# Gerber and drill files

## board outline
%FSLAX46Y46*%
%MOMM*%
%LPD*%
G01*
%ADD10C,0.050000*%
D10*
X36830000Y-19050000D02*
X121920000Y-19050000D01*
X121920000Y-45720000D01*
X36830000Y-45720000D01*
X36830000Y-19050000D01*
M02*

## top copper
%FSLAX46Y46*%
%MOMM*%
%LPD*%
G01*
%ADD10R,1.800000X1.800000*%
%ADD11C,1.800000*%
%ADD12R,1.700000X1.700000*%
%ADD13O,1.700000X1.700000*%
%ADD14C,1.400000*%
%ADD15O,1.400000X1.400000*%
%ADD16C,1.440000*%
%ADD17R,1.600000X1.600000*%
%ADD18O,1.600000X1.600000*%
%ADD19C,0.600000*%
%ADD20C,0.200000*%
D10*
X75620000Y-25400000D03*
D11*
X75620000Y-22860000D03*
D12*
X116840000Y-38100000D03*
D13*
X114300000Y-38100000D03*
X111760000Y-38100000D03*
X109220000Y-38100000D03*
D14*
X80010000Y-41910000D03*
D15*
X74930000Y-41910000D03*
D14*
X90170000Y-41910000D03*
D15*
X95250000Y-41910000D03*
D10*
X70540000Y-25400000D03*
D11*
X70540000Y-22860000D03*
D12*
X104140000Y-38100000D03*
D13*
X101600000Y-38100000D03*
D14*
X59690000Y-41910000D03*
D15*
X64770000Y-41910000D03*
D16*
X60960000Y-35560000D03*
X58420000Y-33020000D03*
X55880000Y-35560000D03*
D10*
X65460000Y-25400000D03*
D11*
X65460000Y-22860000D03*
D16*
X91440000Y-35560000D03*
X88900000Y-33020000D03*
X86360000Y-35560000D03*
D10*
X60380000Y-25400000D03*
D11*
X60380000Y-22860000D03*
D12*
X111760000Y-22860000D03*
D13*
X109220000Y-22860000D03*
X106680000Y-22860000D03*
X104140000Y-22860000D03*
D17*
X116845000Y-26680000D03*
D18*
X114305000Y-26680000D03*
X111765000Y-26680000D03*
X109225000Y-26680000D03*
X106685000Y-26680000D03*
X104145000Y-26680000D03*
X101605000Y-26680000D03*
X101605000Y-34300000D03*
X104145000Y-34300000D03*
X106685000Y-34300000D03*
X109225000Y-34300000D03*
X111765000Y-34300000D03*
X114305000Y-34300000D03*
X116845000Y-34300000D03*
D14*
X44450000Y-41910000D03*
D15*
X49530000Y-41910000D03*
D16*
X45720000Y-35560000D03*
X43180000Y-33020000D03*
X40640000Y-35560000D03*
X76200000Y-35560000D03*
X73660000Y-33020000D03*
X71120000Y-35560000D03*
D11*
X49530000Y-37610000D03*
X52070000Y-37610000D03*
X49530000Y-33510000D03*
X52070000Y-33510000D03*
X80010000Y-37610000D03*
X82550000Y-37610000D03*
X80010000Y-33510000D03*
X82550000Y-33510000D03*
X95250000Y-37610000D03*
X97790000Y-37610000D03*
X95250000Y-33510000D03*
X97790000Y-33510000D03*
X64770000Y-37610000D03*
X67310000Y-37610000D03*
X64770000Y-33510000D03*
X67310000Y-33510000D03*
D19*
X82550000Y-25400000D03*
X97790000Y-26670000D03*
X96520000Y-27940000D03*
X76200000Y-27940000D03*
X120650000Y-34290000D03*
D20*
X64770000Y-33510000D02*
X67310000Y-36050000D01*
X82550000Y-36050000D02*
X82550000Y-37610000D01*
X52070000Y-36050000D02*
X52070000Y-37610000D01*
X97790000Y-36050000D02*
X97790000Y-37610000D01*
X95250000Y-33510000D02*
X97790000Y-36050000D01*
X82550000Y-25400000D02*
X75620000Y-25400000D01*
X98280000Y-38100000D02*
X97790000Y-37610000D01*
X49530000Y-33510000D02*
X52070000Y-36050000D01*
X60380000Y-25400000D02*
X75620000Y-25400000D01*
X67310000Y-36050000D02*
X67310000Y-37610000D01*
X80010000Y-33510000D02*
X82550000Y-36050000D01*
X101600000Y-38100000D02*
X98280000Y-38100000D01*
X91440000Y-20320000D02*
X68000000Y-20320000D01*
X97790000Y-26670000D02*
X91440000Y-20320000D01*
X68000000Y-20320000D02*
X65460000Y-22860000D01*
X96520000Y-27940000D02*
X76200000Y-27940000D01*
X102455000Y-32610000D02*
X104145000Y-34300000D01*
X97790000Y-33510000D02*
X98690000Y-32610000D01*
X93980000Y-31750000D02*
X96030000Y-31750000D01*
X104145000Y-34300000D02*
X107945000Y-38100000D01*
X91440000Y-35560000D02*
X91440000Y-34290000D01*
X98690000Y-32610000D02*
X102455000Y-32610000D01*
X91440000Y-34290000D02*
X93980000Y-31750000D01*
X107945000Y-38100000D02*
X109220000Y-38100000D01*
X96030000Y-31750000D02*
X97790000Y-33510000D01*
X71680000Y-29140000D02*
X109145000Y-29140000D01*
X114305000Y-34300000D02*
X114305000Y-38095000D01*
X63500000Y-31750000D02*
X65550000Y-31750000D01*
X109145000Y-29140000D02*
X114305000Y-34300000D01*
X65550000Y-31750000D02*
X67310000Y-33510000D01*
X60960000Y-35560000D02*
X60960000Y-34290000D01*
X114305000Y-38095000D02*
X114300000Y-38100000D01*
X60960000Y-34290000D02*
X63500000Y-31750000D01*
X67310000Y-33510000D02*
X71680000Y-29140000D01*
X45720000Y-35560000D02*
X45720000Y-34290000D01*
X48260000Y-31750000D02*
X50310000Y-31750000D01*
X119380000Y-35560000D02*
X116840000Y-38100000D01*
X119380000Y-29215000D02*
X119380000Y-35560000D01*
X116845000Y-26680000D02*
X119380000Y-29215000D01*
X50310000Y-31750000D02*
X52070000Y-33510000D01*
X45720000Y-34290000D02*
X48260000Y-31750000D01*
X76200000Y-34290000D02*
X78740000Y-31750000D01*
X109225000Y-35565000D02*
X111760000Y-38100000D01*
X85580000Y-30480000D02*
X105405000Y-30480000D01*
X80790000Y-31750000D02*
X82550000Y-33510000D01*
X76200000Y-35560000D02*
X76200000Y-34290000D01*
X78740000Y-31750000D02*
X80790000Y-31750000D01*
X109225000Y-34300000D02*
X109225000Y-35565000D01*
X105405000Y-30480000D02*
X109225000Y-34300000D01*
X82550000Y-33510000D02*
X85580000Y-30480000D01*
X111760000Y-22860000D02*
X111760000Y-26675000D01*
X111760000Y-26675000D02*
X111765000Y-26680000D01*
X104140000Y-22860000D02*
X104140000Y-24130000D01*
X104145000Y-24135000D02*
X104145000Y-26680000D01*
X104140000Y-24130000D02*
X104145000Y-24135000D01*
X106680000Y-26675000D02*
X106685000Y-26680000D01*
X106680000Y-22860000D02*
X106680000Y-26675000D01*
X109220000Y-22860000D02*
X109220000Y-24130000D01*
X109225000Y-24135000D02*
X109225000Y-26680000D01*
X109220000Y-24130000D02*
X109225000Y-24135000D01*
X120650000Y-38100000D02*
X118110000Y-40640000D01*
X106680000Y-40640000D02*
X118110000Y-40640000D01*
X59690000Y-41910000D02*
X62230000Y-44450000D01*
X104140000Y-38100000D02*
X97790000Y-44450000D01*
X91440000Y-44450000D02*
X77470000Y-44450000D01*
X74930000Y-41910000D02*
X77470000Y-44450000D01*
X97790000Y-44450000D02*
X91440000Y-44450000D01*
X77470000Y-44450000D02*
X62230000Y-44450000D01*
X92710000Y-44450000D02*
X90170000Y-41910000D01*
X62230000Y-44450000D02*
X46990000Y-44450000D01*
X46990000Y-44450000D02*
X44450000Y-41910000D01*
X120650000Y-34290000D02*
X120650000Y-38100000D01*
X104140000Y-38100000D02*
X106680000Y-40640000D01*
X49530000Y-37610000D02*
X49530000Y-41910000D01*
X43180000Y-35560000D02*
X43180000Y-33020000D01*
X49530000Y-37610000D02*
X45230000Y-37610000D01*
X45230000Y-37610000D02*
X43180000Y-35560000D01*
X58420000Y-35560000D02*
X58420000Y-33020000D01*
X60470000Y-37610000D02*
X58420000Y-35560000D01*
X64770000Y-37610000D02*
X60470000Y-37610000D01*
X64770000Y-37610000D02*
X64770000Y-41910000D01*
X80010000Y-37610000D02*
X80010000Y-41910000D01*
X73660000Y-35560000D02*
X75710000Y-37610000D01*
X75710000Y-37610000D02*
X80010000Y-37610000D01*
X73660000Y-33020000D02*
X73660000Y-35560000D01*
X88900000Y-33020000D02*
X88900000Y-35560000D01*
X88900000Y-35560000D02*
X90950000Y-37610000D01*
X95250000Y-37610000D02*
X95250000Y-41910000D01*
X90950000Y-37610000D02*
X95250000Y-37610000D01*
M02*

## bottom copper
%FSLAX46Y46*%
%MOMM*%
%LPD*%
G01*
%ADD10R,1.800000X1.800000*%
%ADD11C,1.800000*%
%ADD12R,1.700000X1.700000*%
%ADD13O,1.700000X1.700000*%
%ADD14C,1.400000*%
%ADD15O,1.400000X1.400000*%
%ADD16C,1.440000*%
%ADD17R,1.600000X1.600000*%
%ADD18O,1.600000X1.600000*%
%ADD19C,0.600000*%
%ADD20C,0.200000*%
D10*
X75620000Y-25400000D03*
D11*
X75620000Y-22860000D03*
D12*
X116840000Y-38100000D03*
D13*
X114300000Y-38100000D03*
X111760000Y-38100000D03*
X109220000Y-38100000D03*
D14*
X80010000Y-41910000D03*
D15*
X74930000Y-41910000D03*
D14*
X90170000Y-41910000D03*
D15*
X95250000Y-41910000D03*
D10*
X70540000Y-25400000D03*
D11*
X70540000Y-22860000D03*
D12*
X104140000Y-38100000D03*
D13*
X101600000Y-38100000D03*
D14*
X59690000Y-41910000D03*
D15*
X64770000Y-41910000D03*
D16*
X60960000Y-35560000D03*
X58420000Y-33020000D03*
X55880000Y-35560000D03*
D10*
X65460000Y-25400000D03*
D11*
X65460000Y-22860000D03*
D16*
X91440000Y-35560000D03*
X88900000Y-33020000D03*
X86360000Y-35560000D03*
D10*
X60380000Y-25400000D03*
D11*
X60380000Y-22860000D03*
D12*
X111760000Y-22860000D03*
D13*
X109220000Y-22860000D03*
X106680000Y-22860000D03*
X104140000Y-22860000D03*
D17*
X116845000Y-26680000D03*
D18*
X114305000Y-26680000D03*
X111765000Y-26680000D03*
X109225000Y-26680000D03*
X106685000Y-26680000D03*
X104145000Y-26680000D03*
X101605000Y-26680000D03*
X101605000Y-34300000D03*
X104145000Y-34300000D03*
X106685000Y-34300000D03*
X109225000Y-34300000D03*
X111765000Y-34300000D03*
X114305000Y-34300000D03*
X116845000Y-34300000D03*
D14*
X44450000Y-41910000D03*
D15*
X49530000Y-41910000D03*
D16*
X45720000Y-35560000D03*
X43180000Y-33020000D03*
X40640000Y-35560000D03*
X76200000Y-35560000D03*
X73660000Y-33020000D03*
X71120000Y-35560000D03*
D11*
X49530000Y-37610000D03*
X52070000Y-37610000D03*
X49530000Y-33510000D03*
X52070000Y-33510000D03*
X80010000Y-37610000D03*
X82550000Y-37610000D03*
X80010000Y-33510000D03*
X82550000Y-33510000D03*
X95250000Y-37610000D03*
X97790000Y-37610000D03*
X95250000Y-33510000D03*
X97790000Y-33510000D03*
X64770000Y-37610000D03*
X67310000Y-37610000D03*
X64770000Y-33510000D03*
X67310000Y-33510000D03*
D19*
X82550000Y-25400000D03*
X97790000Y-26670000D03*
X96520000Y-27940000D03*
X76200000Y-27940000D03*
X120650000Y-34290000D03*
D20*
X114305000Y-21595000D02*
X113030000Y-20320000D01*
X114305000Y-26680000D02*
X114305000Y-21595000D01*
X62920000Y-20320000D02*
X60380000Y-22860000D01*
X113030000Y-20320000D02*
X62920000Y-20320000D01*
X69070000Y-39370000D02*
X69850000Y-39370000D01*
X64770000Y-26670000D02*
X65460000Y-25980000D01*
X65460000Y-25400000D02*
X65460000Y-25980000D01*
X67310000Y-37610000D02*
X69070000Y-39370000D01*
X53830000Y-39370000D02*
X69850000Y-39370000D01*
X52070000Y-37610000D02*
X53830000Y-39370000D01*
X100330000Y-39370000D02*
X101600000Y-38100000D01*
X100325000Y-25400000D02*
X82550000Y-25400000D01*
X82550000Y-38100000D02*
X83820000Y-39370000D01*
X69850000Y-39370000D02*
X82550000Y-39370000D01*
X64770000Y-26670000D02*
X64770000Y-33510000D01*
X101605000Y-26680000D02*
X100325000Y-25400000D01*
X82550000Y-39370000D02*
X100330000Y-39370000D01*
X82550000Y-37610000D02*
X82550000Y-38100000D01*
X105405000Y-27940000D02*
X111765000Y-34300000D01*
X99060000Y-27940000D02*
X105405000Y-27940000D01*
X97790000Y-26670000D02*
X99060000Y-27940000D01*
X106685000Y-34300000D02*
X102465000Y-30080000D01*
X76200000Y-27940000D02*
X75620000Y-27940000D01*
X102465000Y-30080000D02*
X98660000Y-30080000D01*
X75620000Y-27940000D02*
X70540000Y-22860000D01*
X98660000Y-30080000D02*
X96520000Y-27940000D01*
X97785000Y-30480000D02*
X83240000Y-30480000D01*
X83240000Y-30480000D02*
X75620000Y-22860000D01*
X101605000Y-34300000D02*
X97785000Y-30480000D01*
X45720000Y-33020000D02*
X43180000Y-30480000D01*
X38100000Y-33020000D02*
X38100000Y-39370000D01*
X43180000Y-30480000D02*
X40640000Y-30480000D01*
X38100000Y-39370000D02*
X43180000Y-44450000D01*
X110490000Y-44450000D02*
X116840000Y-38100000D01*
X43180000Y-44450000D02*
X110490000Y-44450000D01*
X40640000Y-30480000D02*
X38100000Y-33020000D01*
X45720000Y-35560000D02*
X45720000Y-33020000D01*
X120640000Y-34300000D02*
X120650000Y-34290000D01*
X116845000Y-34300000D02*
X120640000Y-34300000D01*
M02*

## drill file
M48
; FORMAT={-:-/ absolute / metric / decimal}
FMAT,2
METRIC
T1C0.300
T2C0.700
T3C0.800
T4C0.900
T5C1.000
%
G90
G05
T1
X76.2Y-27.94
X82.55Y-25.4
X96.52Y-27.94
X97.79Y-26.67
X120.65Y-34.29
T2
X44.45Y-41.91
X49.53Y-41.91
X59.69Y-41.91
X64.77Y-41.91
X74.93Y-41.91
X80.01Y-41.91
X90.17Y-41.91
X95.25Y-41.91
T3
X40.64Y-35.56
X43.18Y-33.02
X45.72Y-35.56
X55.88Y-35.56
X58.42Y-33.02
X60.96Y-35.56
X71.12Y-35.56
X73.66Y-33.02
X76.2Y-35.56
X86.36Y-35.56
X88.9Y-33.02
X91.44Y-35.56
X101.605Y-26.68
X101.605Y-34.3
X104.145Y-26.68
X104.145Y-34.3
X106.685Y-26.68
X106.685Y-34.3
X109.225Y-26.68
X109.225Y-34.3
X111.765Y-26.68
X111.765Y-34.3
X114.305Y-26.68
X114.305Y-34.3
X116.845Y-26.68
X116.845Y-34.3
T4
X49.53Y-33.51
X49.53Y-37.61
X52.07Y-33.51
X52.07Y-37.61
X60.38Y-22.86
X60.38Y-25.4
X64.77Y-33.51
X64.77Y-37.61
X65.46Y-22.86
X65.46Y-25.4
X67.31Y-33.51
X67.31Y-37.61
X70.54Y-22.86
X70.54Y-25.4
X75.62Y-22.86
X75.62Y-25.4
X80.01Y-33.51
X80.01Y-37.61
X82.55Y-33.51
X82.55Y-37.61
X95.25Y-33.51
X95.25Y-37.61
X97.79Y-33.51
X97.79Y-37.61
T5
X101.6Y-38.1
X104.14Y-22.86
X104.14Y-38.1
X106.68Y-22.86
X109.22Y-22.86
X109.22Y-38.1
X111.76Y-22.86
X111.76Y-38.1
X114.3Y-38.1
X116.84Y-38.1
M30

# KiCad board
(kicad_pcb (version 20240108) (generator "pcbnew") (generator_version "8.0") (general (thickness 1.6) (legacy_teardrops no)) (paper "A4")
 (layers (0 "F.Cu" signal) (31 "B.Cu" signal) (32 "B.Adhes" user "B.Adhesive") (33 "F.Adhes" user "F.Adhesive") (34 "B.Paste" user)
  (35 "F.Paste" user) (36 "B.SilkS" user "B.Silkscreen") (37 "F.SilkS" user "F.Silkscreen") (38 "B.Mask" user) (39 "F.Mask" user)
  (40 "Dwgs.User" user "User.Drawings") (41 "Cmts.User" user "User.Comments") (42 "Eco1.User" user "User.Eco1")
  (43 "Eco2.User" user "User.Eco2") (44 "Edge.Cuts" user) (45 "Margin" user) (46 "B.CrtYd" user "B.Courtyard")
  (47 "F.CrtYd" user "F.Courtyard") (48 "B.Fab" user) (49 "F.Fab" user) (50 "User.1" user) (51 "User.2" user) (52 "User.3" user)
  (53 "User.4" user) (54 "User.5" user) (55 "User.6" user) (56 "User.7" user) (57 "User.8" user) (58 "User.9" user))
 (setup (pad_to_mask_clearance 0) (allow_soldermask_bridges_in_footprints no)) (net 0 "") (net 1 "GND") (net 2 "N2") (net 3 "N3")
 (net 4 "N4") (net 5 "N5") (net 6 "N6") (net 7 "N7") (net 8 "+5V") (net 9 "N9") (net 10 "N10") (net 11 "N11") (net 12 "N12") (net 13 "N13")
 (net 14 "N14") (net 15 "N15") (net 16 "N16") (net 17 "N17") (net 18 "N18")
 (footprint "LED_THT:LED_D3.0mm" (layer "F.Cu") (at 75.62 25.4 90)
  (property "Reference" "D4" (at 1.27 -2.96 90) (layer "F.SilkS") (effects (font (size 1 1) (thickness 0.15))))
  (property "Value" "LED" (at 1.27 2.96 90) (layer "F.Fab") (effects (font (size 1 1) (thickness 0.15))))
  (pad "1" thru_hole rect (at 0 0 90) (size 1.8 1.8) (drill 0.9) (layers "*.Cu" "*.Mask") (remove_unused_layers no) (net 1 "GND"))
  (pad "2" thru_hole circle (at 2.54 0 90) (size 1.8 1.8) (drill 0.9) (layers "*.Cu" "*.Mask") (remove_unused_layers no) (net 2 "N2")))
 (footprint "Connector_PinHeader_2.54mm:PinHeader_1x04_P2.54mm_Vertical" (layer "F.Cu") (at 116.84 38.1 -90)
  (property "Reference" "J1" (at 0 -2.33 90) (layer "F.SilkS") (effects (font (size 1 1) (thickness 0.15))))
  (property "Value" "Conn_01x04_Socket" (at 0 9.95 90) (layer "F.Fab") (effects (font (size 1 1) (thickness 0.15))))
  (pad "1" thru_hole rect (at 0 0 270) (size 1.7 1.7) (drill 1) (layers "*.Cu" "*.Mask") (remove_unused_layers no) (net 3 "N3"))
  (pad "2" thru_hole oval (at 0 2.54 270) (size 1.7 1.7) (drill 1) (layers "*.Cu" "*.Mask") (remove_unused_layers no) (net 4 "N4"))
  (pad "3" thru_hole oval (at 0 5.08 270) (size 1.7 1.7) (drill 1) (layers "*.Cu" "*.Mask") (remove_unused_layers no) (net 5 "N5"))
  (pad "4" thru_hole oval (at 0 7.62 270) (size 1.7 1.7) (drill 1) (layers "*.Cu" "*.Mask") (remove_unused_layers no) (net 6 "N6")))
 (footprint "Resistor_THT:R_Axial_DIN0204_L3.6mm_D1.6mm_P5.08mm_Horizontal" (layer "F.Cu") (at 80.01 41.91 180)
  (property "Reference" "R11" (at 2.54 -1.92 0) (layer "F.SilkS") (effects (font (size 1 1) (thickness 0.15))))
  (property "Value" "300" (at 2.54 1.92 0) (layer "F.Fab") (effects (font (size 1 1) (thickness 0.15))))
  (pad "1" thru_hole circle (at 0 0 180) (size 1.4 1.4) (drill 0.7) (layers "*.Cu" "*.Mask") (remove_unused_layers no) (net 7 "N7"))
  (pad "2" thru_hole oval (at 5.08 0 180) (size 1.4 1.4) (drill 0.7) (layers "*.Cu" "*.Mask") (remove_unused_layers no) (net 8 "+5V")))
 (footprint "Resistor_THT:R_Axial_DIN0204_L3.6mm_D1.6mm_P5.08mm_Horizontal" (layer "F.Cu") (at 90.17 41.91)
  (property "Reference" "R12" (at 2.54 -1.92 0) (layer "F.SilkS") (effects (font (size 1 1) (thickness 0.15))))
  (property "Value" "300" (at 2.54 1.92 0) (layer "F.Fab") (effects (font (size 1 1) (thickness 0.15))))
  (pad "1" thru_hole circle (at 0 0) (size 1.4 1.4) (drill 0.7) (layers "*.Cu" "*.Mask") (remove_unused_layers no) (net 8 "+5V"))
  (pad "2" thru_hole oval (at 5.08 0) (size 1.4 1.4) (drill 0.7) (layers "*.Cu" "*.Mask") (remove_unused_layers no) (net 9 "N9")))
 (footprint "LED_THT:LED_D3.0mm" (layer "F.Cu") (at 70.54 25.4 90)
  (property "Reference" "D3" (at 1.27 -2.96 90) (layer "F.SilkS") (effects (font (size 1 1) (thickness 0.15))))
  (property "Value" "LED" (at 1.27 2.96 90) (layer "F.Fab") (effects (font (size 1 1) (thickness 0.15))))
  (pad "1" thru_hole rect (at 0 0 90) (size 1.8 1.8) (drill 0.9) (layers "*.Cu" "*.Mask") (remove_unused_layers no) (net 1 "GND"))
  (pad "2" thru_hole circle (at 2.54 0 90) (size 1.8 1.8) (drill 0.9) (layers "*.Cu" "*.Mask") (remove_unused_layers no) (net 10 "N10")))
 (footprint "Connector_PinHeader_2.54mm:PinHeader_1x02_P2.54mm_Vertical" (layer "F.Cu") (at 104.14 38.1 -90)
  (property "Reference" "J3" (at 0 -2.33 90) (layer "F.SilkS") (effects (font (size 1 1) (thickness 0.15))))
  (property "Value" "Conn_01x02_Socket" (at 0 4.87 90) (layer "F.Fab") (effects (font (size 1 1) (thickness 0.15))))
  (pad "1" thru_hole rect (at 0 0 270) (size 1.7 1.7) (drill 1) (layers "*.Cu" "*.Mask") (remove_unused_layers no) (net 8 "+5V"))
  (pad "2" thru_hole oval (at 0 2.54 270) (size 1.7 1.7) (drill 1) (layers "*.Cu" "*.Mask") (remove_unused_layers no) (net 1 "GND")))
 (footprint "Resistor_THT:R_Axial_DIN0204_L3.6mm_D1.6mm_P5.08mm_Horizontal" (layer "F.Cu") (at 59.69 41.91)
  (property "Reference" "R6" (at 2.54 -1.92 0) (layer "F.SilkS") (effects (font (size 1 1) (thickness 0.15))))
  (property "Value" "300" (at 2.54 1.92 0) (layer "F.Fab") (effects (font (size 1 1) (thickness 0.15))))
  (pad "1" thru_hole circle (at 0 0) (size 1.4 1.4) (drill 0.7) (layers "*.Cu" "*.Mask") (remove_unused_layers no) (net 8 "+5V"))
  (pad "2" thru_hole oval (at 5.08 0) (size 1.4 1.4) (drill 0.7) (layers "*.Cu" "*.Mask") (remove_unused_layers no) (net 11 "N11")))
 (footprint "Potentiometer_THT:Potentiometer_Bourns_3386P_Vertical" (layer "F.Cu") (at 60.96 35.56 90)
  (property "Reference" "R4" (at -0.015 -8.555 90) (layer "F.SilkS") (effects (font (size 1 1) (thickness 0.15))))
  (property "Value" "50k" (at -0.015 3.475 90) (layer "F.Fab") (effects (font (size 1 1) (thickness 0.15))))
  (pad "1" thru_hole circle (at 0 0 90) (size 1.44 1.44) (drill 0.8) (layers "*.Cu" "*.Mask") (remove_unused_layers no) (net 4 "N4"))
  (pad "2" thru_hole circle (at 2.54 -2.54 90) (size 1.44 1.44) (drill 0.8) (layers "*.Cu" "*.Mask") (remove_unused_layers no)
   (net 11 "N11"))
  (pad "3" thru_hole circle (at 0 -5.08 90) (size 1.44 1.44) (drill 0.8) (layers "*.Cu" "*.Mask") (remove_unused_layers no)))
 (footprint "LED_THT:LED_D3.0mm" (layer "F.Cu") (at 65.46 25.4 90)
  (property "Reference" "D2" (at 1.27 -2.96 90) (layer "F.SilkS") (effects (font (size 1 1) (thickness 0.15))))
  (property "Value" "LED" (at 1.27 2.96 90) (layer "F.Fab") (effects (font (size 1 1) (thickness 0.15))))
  (pad "1" thru_hole rect (at 0 0 90) (size 1.8 1.8) (drill 0.9) (layers "*.Cu" "*.Mask") (remove_unused_layers no) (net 1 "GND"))
  (pad "2" thru_hole circle (at 2.54 0 90) (size 1.8 1.8) (drill 0.9) (layers "*.Cu" "*.Mask") (remove_unused_layers no) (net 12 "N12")))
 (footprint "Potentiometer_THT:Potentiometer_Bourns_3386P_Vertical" (layer "F.Cu") (at 91.44 35.56 90)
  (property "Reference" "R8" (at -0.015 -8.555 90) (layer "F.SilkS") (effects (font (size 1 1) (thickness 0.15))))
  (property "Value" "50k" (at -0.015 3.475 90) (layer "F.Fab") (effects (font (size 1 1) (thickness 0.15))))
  (pad "1" thru_hole circle (at 0 0 90) (size 1.44 1.44) (drill 0.8) (layers "*.Cu" "*.Mask") (remove_unused_layers no) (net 6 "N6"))
  (pad "2" thru_hole circle (at 2.54 -2.54 90) (size 1.44 1.44) (drill 0.8) (layers "*.Cu" "*.Mask") (remove_unused_layers no) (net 9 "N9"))
  (pad "3" thru_hole circle (at 0 -5.08 90) (size 1.44 1.44) (drill 0.8) (layers "*.Cu" "*.Mask") (remove_unused_layers no)))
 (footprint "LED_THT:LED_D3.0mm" (layer "F.Cu") (at 60.38 25.4 90)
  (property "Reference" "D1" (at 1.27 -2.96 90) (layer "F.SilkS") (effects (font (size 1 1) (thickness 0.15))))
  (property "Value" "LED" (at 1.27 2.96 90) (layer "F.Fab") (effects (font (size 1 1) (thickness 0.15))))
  (pad "1" thru_hole rect (at 0 0 90) (size 1.8 1.8) (drill 0.9) (layers "*.Cu" "*.Mask") (remove_unused_layers no) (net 1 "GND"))
  (pad "2" thru_hole circle (at 2.54 0 90) (size 1.8 1.8) (drill 0.9) (layers "*.Cu" "*.Mask") (remove_unused_layers no) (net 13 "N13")))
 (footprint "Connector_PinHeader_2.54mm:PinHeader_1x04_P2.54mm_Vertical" (layer "F.Cu") (at 111.76 22.86 -90)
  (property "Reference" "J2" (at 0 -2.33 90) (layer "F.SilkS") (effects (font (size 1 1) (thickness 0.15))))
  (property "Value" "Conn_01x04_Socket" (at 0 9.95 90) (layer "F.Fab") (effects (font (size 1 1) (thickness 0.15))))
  (pad "1" thru_hole rect (at 0 0 270) (size 1.7 1.7) (drill 1) (layers "*.Cu" "*.Mask") (remove_unused_layers no) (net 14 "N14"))
  (pad "2" thru_hole oval (at 0 2.54 270) (size 1.7 1.7) (drill 1) (layers "*.Cu" "*.Mask") (remove_unused_layers no) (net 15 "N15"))
  (pad "3" thru_hole oval (at 0 5.08 270) (size 1.7 1.7) (drill 1) (layers "*.Cu" "*.Mask") (remove_unused_layers no) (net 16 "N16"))
  (pad "4" thru_hole oval (at 0 7.62 270) (size 1.7 1.7) (drill 1) (layers "*.Cu" "*.Mask") (remove_unused_layers no) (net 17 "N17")))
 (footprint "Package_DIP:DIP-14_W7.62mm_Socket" (layer "F.Cu") (at 116.845 26.68 -90)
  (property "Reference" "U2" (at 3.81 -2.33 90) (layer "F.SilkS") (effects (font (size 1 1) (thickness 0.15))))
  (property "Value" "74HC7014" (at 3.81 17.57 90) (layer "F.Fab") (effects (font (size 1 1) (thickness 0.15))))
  (pad "1" thru_hole rect (at 0 0 270) (size 1.6 1.6) (drill 0.8) (layers "*.Cu" "*.Mask") (remove_unused_layers no) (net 3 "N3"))
  (pad "2" thru_hole oval (at 0 2.54 270) (size 1.6 1.6) (drill 0.8) (layers "*.Cu" "*.Mask") (remove_unused_layers no) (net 13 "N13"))
  (pad "3" thru_hole oval (at 0 5.08 270) (size 1.6 1.6) (drill 0.8) (layers "*.Cu" "*.Mask") (remove_unused_layers no) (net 14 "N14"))
  (pad "4" thru_hole oval (at 0 7.62 270) (size 1.6 1.6) (drill 0.8) (layers "*.Cu" "*.Mask") (remove_unused_layers no) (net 15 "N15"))
  (pad "5" thru_hole oval (at 0 10.16 270) (size 1.6 1.6) (drill 0.8) (layers "*.Cu" "*.Mask") (remove_unused_layers no) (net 16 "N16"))
  (pad "6" thru_hole oval (at 0 12.7 270) (size 1.6 1.6) (drill 0.8) (layers "*.Cu" "*.Mask") (remove_unused_layers no) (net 17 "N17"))
  (pad "7" thru_hole oval (at 0 15.24 270) (size 1.6 1.6) (drill 0.8) (layers "*.Cu" "*.Mask") (remove_unused_layers no) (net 1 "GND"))
  (pad "8" thru_hole oval (at 7.62 15.24 270) (size 1.6 1.6) (drill 0.8) (layers "*.Cu" "*.Mask") (remove_unused_layers no) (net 2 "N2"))
  (pad "9" thru_hole oval (at 7.62 12.7 270) (size 1.6 1.6) (drill 0.8) (layers "*.Cu" "*.Mask") (remove_unused_layers no) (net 6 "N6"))
  (pad "10" thru_hole oval (at 7.62 10.16 270) (size 1.6 1.6) (drill 0.8) (layers "*.Cu" "*.Mask") (remove_unused_layers no) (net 10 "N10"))
  (pad "11" thru_hole oval (at 7.62 7.62 270) (size 1.6 1.6) (drill 0.8) (layers "*.Cu" "*.Mask") (remove_unused_layers no) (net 5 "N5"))
  (pad "12" thru_hole oval (at 7.62 5.08 270) (size 1.6 1.6) (drill 0.8) (layers "*.Cu" "*.Mask") (remove_unused_layers no) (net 12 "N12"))
  (pad "13" thru_hole oval (at 7.62 2.54 270) (size 1.6 1.6) (drill 0.8) (layers "*.Cu" "*.Mask") (remove_unused_layers no) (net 4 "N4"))
  (pad "14" thru_hole oval (at 7.62 0 270) (size 1.6 1.6) (drill 0.8) (layers "*.Cu" "*.Mask") (remove_unused_layers no) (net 8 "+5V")))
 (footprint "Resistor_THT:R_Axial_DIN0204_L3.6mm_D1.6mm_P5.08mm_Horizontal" (layer "F.Cu") (at 44.45 41.91)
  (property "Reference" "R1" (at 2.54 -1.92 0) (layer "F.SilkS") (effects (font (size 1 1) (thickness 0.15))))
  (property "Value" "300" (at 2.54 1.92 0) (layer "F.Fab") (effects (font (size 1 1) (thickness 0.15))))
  (pad "1" thru_hole circle (at 0 0) (size 1.4 1.4) (drill 0.7) (layers "*.Cu" "*.Mask") (remove_unused_layers no) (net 8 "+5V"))
  (pad "2" thru_hole oval (at 5.08 0) (size 1.4 1.4) (drill 0.7) (layers "*.Cu" "*.Mask") (remove_unused_layers no) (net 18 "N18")))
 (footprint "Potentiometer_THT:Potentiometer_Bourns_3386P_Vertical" (layer "F.Cu") (at 45.72 35.56 90)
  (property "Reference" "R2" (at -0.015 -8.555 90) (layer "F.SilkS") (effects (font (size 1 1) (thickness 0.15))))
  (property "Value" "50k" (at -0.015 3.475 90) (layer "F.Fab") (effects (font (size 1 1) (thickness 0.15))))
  (pad "1" thru_hole circle (at 0 0 90) (size 1.44 1.44) (drill 0.8) (layers "*.Cu" "*.Mask") (remove_unused_layers no) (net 3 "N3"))
  (pad "2" thru_hole circle (at 2.54 -2.54 90) (size 1.44 1.44) (drill 0.8) (layers "*.Cu" "*.Mask") (remove_unused_layers no)
   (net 18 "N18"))
  (pad "3" thru_hole circle (at 0 -5.08 90) (size 1.44 1.44) (drill 0.8) (layers "*.Cu" "*.Mask") (remove_unused_layers no)))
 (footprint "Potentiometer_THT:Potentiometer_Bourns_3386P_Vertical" (layer "F.Cu") (at 76.2 35.56 90)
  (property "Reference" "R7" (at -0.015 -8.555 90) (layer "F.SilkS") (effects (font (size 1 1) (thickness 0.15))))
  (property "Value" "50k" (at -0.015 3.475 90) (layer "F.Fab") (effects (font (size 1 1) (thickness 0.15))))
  (pad "1" thru_hole circle (at 0 0 90) (size 1.44 1.44) (drill 0.8) (layers "*.Cu" "*.Mask") (remove_unused_layers no) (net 5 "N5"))
  (pad "2" thru_hole circle (at 2.54 -2.54 90) (size 1.44 1.44) (drill 0.8) (layers "*.Cu" "*.Mask") (remove_unused_layers no) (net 7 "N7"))
  (pad "3" thru_hole circle (at 0 -5.08 90) (size 1.44 1.44) (drill 0.8) (layers "*.Cu" "*.Mask") (remove_unused_layers no)))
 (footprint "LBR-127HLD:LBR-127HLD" (layer "B.Cu") (at 50.8 35.56 -90)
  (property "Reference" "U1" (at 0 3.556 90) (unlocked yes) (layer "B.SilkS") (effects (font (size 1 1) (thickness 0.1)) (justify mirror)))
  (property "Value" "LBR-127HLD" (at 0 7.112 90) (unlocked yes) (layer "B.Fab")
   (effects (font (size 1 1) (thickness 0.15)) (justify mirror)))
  (pad "1" thru_hole circle (at 2.05 1.27 270) (size 1.8 1.8) (drill 0.9) (layers "*.Cu" "*.Mask") (remove_unused_layers no) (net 18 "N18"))
  (pad "2" thru_hole circle (at 2.05 -1.27 270) (size 1.8 1.8) (drill 0.9) (layers "*.Cu" "*.Mask") (remove_unused_layers no) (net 1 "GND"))
  (pad "3" thru_hole circle (at -2.05 1.27 270) (size 1.8 1.8) (drill 0.9) (layers "*.Cu" "*.Mask") (remove_unused_layers no) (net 1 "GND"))
  (pad "4" thru_hole circle (at -2.05 -1.27 270) (size 1.8 1.8) (drill 0.9) (layers "*.Cu" "*.Mask") (remove_unused_layers no) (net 3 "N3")))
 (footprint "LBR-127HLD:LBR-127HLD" (layer "B.Cu") (at 81.28 35.56 -90)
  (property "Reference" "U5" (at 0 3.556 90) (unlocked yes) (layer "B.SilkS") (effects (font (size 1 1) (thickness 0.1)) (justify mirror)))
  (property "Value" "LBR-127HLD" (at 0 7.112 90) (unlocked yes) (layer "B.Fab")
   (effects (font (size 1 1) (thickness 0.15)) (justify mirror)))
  (pad "1" thru_hole circle (at 2.05 1.27 270) (size 1.8 1.8) (drill 0.9) (layers "*.Cu" "*.Mask") (remove_unused_layers no) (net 7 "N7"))
  (pad "2" thru_hole circle (at 2.05 -1.27 270) (size 1.8 1.8) (drill 0.9) (layers "*.Cu" "*.Mask") (remove_unused_layers no) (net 1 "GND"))
  (pad "3" thru_hole circle (at -2.05 1.27 270) (size 1.8 1.8) (drill 0.9) (layers "*.Cu" "*.Mask") (remove_unused_layers no) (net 1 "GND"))
  (pad "4" thru_hole circle (at -2.05 -1.27 270) (size 1.8 1.8) (drill 0.9) (layers "*.Cu" "*.Mask") (remove_unused_layers no) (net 5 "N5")))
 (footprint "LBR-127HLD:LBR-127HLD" (layer "B.Cu") (at 96.52 35.56 -90)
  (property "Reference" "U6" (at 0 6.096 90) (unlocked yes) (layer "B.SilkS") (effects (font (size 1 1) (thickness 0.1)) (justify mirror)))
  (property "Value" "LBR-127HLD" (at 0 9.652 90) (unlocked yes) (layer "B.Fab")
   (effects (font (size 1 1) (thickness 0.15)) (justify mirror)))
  (pad "1" thru_hole circle (at 2.05 1.27 270) (size 1.8 1.8) (drill 0.9) (layers "*.Cu" "*.Mask") (remove_unused_layers no) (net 9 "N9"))
  (pad "2" thru_hole circle (at 2.05 -1.27 270) (size 1.8 1.8) (drill 0.9) (layers "*.Cu" "*.Mask") (remove_unused_layers no) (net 1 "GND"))
  (pad "3" thru_hole circle (at -2.05 1.27 270) (size 1.8 1.8) (drill 0.9) (layers "*.Cu" "*.Mask") (remove_unused_layers no) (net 1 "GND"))
  (pad "4" thru_hole circle (at -2.05 -1.27 270) (size 1.8 1.8) (drill 0.9) (layers "*.Cu" "*.Mask") (remove_unused_layers no) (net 6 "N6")))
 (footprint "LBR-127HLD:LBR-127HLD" (layer "B.Cu") (at 66.04 35.56 -90)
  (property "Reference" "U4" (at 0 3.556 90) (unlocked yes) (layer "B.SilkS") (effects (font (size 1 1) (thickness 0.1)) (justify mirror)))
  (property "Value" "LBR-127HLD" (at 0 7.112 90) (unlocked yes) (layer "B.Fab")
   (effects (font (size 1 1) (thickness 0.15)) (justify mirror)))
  (pad "1" thru_hole circle (at 2.05 1.27 270) (size 1.8 1.8) (drill 0.9) (layers "*.Cu" "*.Mask") (remove_unused_layers no) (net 11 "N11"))
  (pad "2" thru_hole circle (at 2.05 -1.27 270) (size 1.8 1.8) (drill 0.9) (layers "*.Cu" "*.Mask") (remove_unused_layers no) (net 1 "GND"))
  (pad "3" thru_hole circle (at -2.05 1.27 270) (size 1.8 1.8) (drill 0.9) (layers "*.Cu" "*.Mask") (remove_unused_layers no) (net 1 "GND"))
  (pad "4" thru_hole circle (at -2.05 -1.27 270) (size 1.8 1.8) (drill 0.9) (layers "*.Cu" "*.Mask") (remove_unused_layers no) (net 4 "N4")))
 (gr_rect (start 36.83 19.05) (end 121.92 45.72) (stroke (width 0.05) (type default)) (fill none) (layer "Edge.Cuts"))
 (segment (start 114.305 21.595) (end 113.03 20.32) (width 0.2) (layer "B.Cu") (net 13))
 (segment (start 114.305 26.68) (end 114.305 21.595) (width 0.2) (layer "B.Cu") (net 13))
 (segment (start 62.92 20.32) (end 60.38 22.86) (width 0.2) (layer "B.Cu") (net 13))
 (segment (start 113.03 20.32) (end 62.92 20.32) (width 0.2) (layer "B.Cu") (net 13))
 (segment (start 64.77 33.51) (end 67.31 36.05) (width 0.2) (layer "F.Cu") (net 1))
 (segment (start 82.55 36.05) (end 82.55 37.61) (width 0.2) (layer "F.Cu") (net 1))
 (segment (start 52.07 36.05) (end 52.07 37.61) (width 0.2) (layer "F.Cu") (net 1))
 (segment (start 97.79 36.05) (end 97.79 37.61) (width 0.2) (layer "F.Cu") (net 1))
 (segment (start 95.25 33.51) (end 97.79 36.05) (width 0.2) (layer "F.Cu") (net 1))
 (segment (start 82.55 25.4) (end 75.62 25.4) (width 0.2) (layer "F.Cu") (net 1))
 (segment (start 98.28 38.1) (end 97.79 37.61) (width 0.2) (layer "F.Cu") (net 1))
 (segment (start 49.53 33.51) (end 52.07 36.05) (width 0.2) (layer "F.Cu") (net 1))
 (segment (start 60.38 25.4) (end 75.62 25.4) (width 0.2) (layer "F.Cu") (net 1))
 (segment (start 67.31 36.05) (end 67.31 37.61) (width 0.2) (layer "F.Cu") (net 1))
 (segment (start 80.01 33.51) (end 82.55 36.05) (width 0.2) (layer "F.Cu") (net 1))
 (segment (start 101.6 38.1) (end 98.28 38.1) (width 0.2) (layer "F.Cu") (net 1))
 (via (at 82.55 25.4) (size 0.6) (drill 0.3) (layers "F.Cu" "B.Cu") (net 1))
 (segment (start 69.07 39.37) (end 69.85 39.37) (width 0.2) (layer "B.Cu") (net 1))
 (segment (start 64.77 26.67) (end 65.46 25.98) (width 0.2) (layer "B.Cu") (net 1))
 (segment (start 65.46 25.4) (end 65.46 25.98) (width 0.2) (layer "B.Cu") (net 1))
 (segment (start 67.31 37.61) (end 69.07 39.37) (width 0.2) (layer "B.Cu") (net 1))
 (segment (start 53.83 39.37) (end 69.85 39.37) (width 0.2) (layer "B.Cu") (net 1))
 (segment (start 52.07 37.61) (end 53.83 39.37) (width 0.2) (layer "B.Cu") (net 1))
 (segment (start 100.33 39.37) (end 101.6 38.1) (width 0.2) (layer "B.Cu") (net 1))
 (segment (start 100.325 25.4) (end 82.55 25.4) (width 0.2) (layer "B.Cu") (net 1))
 (segment (start 82.55 38.1) (end 83.82 39.37) (width 0.2) (layer "B.Cu") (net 1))
 (segment (start 69.85 39.37) (end 82.55 39.37) (width 0.2) (layer "B.Cu") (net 1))
 (segment (start 64.77 26.67) (end 64.77 33.51) (width 0.2) (layer "B.Cu") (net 1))
 (segment (start 101.605 26.68) (end 100.325 25.4) (width 0.2) (layer "B.Cu") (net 1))
 (segment (start 82.55 39.37) (end 100.33 39.37) (width 0.2) (layer "B.Cu") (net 1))
 (segment (start 82.55 37.61) (end 82.55 38.1) (width 0.2) (layer "B.Cu") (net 1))
 (segment (start 91.44 20.32) (end 68 20.32) (width 0.2) (layer "F.Cu") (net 12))
 (segment (start 97.79 26.67) (end 91.44 20.32) (width 0.2) (layer "F.Cu") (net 12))
 (segment (start 68 20.32) (end 65.46 22.86) (width 0.2) (layer "F.Cu") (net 12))
 (via (at 97.79 26.67) (size 0.6) (drill 0.3) (layers "F.Cu" "B.Cu") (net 12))
 (segment (start 105.405 27.94) (end 111.765 34.3) (width 0.2) (layer "B.Cu") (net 12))
 (segment (start 99.06 27.94) (end 105.405 27.94) (width 0.2) (layer "B.Cu") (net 12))
 (segment (start 97.79 26.67) (end 99.06 27.94) (width 0.2) (layer "B.Cu") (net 12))
 (segment (start 96.52 27.94) (end 76.2 27.94) (width 0.2) (layer "F.Cu") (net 10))
 (via (at 96.52 27.94) (size 0.6) (drill 0.3) (layers "F.Cu" "B.Cu") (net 10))
 (via (at 76.2 27.94) (size 0.6) (drill 0.3) (layers "F.Cu" "B.Cu") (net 10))
 (segment (start 106.685 34.3) (end 102.465 30.08) (width 0.2) (layer "B.Cu") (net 10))
 (segment (start 76.2 27.94) (end 75.62 27.94) (width 0.2) (layer "B.Cu") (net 10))
 (segment (start 102.465 30.08) (end 98.66 30.08) (width 0.2) (layer "B.Cu") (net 10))
 (segment (start 75.62 27.94) (end 70.54 22.86) (width 0.2) (layer "B.Cu") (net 10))
 (segment (start 98.66 30.08) (end 96.52 27.94) (width 0.2) (layer "B.Cu") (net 10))
 (segment (start 97.785 30.48) (end 83.24 30.48) (width 0.2) (layer "B.Cu") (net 2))
 (segment (start 83.24 30.48) (end 75.62 22.86) (width 0.2) (layer "B.Cu") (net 2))
 (segment (start 101.605 34.3) (end 97.785 30.48) (width 0.2) (layer "B.Cu") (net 2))
 (segment (start 102.455 32.61) (end 104.145 34.3) (width 0.2) (layer "F.Cu") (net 6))
 (segment (start 97.79 33.51) (end 98.69 32.61) (width 0.2) (layer "F.Cu") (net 6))
 (segment (start 93.98 31.75) (end 96.03 31.75) (width 0.2) (layer "F.Cu") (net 6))
 (segment (start 104.145 34.3) (end 107.945 38.1) (width 0.2) (layer "F.Cu") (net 6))
 (segment (start 91.44 35.56) (end 91.44 34.29) (width 0.2) (layer "F.Cu") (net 6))
 (segment (start 98.69 32.61) (end 102.455 32.61) (width 0.2) (layer "F.Cu") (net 6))
 (segment (start 91.44 34.29) (end 93.98 31.75) (width 0.2) (layer "F.Cu") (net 6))
 (segment (start 107.945 38.1) (end 109.22 38.1) (width 0.2) (layer "F.Cu") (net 6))
 (segment (start 96.03 31.75) (end 97.79 33.51) (width 0.2) (layer "F.Cu") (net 6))
 (segment (start 71.68 29.14) (end 109.145 29.14) (width 0.2) (layer "F.Cu") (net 4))
 (segment (start 114.305 34.3) (end 114.305 38.095) (width 0.2) (layer "F.Cu") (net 4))
 (segment (start 63.5 31.75) (end 65.55 31.75) (width 0.2) (layer "F.Cu") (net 4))
 (segment (start 109.145 29.14) (end 114.305 34.3) (width 0.2) (layer "F.Cu") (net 4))
 (segment (start 65.55 31.75) (end 67.31 33.51) (width 0.2) (layer "F.Cu") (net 4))
 (segment (start 60.96 35.56) (end 60.96 34.29) (width 0.2) (layer "F.Cu") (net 4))
 (segment (start 114.305 38.095) (end 114.3 38.1) (width 0.2) (layer "F.Cu") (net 4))
 (segment (start 60.96 34.29) (end 63.5 31.75) (width 0.2) (layer "F.Cu") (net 4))
 (segment (start 67.31 33.51) (end 71.68 29.14) (width 0.2) (layer "F.Cu") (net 4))
 (segment (start 45.72 35.56) (end 45.72 34.29) (width 0.2) (layer "F.Cu") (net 3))
 (segment (start 48.26 31.75) (end 50.31 31.75) (width 0.2) (layer "F.Cu") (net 3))
 (segment (start 119.38 35.56) (end 116.84 38.1) (width 0.2) (layer "F.Cu") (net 3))
 (segment (start 119.38 29.215) (end 119.38 35.56) (width 0.2) (layer "F.Cu") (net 3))
 (segment (start 116.845 26.68) (end 119.38 29.215) (width 0.2) (layer "F.Cu") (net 3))
 (segment (start 50.31 31.75) (end 52.07 33.51) (width 0.2) (layer "F.Cu") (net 3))
 (segment (start 45.72 34.29) (end 48.26 31.75) (width 0.2) (layer "F.Cu") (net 3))
 (segment (start 45.72 33.02) (end 43.18 30.48) (width 0.2) (layer "B.Cu") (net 3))
 (segment (start 38.1 33.02) (end 38.1 39.37) (width 0.2) (layer "B.Cu") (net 3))
 (segment (start 43.18 30.48) (end 40.64 30.48) (width 0.2) (layer "B.Cu") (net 3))
 (segment (start 38.1 39.37) (end 43.18 44.45) (width 0.2) (layer "B.Cu") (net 3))
 (segment (start 110.49 44.45) (end 116.84 38.1) (width 0.2) (layer "B.Cu") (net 3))
 (segment (start 43.18 44.45) (end 110.49 44.45) (width 0.2) (layer "B.Cu") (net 3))
 (segment (start 40.64 30.48) (end 38.1 33.02) (width 0.2) (layer "B.Cu") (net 3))
 (segment (start 45.72 35.56) (end 45.72 33.02) (width 0.2) (layer "B.Cu") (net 3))
 (segment (start 76.2 34.29) (end 78.74 31.75) (width 0.2) (layer "F.Cu") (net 5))
 (segment (start 109.225 35.565) (end 111.76 38.1) (width 0.2) (layer "F.Cu") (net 5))
 (segment (start 85.58 30.48) (end 105.405 30.48) (width 0.2) (layer "F.Cu") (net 5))
 (segment (start 80.79 31.75) (end 82.55 33.51) (width 0.2) (layer "F.Cu") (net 5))
 (segment (start 76.2 35.56) (end 76.2 34.29) (width 0.2) (layer "F.Cu") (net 5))
 (segment (start 78.74 31.75) (end 80.79 31.75) (width 0.2) (layer "F.Cu") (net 5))
 (segment (start 109.225 34.3) (end 109.225 35.565) (width 0.2) (layer "F.Cu") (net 5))
 (segment (start 105.405 30.48) (end 109.225 34.3) (width 0.2) (layer "F.Cu") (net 5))
 (segment (start 82.55 33.51) (end 85.58 30.48) (width 0.2) (layer "F.Cu") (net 5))
 (segment (start 111.76 22.86) (end 111.76 26.675) (width 0.2) (layer "F.Cu") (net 14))
 (segment (start 111.76 26.675) (end 111.765 26.68) (width 0.2) (layer "F.Cu") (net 14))
 (segment (start 104.14 22.86) (end 104.14 24.13) (width 0.2) (layer "F.Cu") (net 17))
 (segment (start 104.145 24.135) (end 104.145 26.68) (width 0.2) (layer "F.Cu") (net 17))
 (segment (start 104.14 24.13) (end 104.145 24.135) (width 0.2) (layer "F.Cu") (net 17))
 (segment (start 106.68 26.675) (end 106.685 26.68) (width 0.2) (layer "F.Cu") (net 16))
 (segment (start 106.68 22.86) (end 106.68 26.675) (width 0.2) (layer "F.Cu") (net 16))
 (segment (start 109.22 22.86) (end 109.22 24.13) (width 0.2) (layer "F.Cu") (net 15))
 (segment (start 109.225 24.135) (end 109.225 26.68) (width 0.2) (layer "F.Cu") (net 15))
 (segment (start 109.22 24.13) (end 109.225 24.135) (width 0.2) (layer "F.Cu") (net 15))
 (segment (start 120.65 38.1) (end 118.11 40.64) (width 0.2) (layer "F.Cu") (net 8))
 (segment (start 106.68 40.64) (end 118.11 40.64) (width 0.2) (layer "F.Cu") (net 8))
 (segment (start 59.69 41.91) (end 62.23 44.45) (width 0.2) (layer "F.Cu") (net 8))
 (segment (start 104.14 38.1) (end 97.79 44.45) (width 0.2) (layer "F.Cu") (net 8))
 (segment (start 91.44 44.45) (end 77.47 44.45) (width 0.2) (layer "F.Cu") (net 8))
 (segment (start 74.93 41.91) (end 77.47 44.45) (width 0.2) (layer "F.Cu") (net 8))
 (segment (start 97.79 44.45) (end 91.44 44.45) (width 0.2) (layer "F.Cu") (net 8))
 (segment (start 77.47 44.45) (end 62.23 44.45) (width 0.2) (layer "F.Cu") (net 8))
 (segment (start 92.71 44.45) (end 90.17 41.91) (width 0.2) (layer "F.Cu") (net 8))
 (segment (start 62.23 44.45) (end 46.99 44.45) (width 0.2) (layer "F.Cu") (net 8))
 (segment (start 46.99 44.45) (end 44.45 41.91) (width 0.2) (layer "F.Cu") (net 8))
 (segment (start 120.65 34.29) (end 120.65 38.1) (width 0.2) (layer "F.Cu") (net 8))
 (segment (start 104.14 38.1) (end 106.68 40.64) (width 0.2) (layer "F.Cu") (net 8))
 (via (at 120.65 34.29) (size 0.6) (drill 0.3) (layers "F.Cu" "B.Cu") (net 8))
 (segment (start 120.64 34.3) (end 120.65 34.29) (width 0.2) (layer "B.Cu") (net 8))
 (segment (start 116.845 34.3) (end 120.64 34.3) (width 0.2) (layer "B.Cu") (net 8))
 (segment (start 49.53 37.61) (end 49.53 41.91) (width 0.2) (layer "F.Cu") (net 18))
 (segment (start 43.18 35.56) (end 43.18 33.02) (width 0.2) (layer "F.Cu") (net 18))
 (segment (start 49.53 37.61) (end 45.23 37.61) (width 0.2) (layer "F.Cu") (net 18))
 (segment (start 45.23 37.61) (end 43.18 35.56) (width 0.2) (layer "F.Cu") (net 18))
 (segment (start 58.42 35.56) (end 58.42 33.02) (width 0.2) (layer "F.Cu") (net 11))
 (segment (start 60.47 37.61) (end 58.42 35.56) (width 0.2) (layer "F.Cu") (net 11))
 (segment (start 64.77 37.61) (end 60.47 37.61) (width 0.2) (layer "F.Cu") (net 11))
 (segment (start 64.77 37.61) (end 64.77 41.91) (width 0.2) (layer "F.Cu") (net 11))
 (segment (start 80.01 37.61) (end 80.01 41.91) (width 0.2) (layer "F.Cu") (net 7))
 (segment (start 73.66 35.56) (end 75.71 37.61) (width 0.2) (layer "F.Cu") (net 7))
 (segment (start 75.71 37.61) (end 80.01 37.61) (width 0.2) (layer "F.Cu") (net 7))
 (segment (start 73.66 33.02) (end 73.66 35.56) (width 0.2) (layer "F.Cu") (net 7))
 (segment (start 88.9 33.02) (end 88.9 35.56) (width 0.2) (layer "F.Cu") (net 9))
 (segment (start 88.9 35.56) (end 90.95 37.61) (width 0.2) (layer "F.Cu") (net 9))
 (segment (start 95.25 37.61) (end 95.25 41.91) (width 0.2) (layer "F.Cu") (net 9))
 (segment (start 90.95 37.61) (end 95.25 37.61) (width 0.2) (layer "F.Cu") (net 9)))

